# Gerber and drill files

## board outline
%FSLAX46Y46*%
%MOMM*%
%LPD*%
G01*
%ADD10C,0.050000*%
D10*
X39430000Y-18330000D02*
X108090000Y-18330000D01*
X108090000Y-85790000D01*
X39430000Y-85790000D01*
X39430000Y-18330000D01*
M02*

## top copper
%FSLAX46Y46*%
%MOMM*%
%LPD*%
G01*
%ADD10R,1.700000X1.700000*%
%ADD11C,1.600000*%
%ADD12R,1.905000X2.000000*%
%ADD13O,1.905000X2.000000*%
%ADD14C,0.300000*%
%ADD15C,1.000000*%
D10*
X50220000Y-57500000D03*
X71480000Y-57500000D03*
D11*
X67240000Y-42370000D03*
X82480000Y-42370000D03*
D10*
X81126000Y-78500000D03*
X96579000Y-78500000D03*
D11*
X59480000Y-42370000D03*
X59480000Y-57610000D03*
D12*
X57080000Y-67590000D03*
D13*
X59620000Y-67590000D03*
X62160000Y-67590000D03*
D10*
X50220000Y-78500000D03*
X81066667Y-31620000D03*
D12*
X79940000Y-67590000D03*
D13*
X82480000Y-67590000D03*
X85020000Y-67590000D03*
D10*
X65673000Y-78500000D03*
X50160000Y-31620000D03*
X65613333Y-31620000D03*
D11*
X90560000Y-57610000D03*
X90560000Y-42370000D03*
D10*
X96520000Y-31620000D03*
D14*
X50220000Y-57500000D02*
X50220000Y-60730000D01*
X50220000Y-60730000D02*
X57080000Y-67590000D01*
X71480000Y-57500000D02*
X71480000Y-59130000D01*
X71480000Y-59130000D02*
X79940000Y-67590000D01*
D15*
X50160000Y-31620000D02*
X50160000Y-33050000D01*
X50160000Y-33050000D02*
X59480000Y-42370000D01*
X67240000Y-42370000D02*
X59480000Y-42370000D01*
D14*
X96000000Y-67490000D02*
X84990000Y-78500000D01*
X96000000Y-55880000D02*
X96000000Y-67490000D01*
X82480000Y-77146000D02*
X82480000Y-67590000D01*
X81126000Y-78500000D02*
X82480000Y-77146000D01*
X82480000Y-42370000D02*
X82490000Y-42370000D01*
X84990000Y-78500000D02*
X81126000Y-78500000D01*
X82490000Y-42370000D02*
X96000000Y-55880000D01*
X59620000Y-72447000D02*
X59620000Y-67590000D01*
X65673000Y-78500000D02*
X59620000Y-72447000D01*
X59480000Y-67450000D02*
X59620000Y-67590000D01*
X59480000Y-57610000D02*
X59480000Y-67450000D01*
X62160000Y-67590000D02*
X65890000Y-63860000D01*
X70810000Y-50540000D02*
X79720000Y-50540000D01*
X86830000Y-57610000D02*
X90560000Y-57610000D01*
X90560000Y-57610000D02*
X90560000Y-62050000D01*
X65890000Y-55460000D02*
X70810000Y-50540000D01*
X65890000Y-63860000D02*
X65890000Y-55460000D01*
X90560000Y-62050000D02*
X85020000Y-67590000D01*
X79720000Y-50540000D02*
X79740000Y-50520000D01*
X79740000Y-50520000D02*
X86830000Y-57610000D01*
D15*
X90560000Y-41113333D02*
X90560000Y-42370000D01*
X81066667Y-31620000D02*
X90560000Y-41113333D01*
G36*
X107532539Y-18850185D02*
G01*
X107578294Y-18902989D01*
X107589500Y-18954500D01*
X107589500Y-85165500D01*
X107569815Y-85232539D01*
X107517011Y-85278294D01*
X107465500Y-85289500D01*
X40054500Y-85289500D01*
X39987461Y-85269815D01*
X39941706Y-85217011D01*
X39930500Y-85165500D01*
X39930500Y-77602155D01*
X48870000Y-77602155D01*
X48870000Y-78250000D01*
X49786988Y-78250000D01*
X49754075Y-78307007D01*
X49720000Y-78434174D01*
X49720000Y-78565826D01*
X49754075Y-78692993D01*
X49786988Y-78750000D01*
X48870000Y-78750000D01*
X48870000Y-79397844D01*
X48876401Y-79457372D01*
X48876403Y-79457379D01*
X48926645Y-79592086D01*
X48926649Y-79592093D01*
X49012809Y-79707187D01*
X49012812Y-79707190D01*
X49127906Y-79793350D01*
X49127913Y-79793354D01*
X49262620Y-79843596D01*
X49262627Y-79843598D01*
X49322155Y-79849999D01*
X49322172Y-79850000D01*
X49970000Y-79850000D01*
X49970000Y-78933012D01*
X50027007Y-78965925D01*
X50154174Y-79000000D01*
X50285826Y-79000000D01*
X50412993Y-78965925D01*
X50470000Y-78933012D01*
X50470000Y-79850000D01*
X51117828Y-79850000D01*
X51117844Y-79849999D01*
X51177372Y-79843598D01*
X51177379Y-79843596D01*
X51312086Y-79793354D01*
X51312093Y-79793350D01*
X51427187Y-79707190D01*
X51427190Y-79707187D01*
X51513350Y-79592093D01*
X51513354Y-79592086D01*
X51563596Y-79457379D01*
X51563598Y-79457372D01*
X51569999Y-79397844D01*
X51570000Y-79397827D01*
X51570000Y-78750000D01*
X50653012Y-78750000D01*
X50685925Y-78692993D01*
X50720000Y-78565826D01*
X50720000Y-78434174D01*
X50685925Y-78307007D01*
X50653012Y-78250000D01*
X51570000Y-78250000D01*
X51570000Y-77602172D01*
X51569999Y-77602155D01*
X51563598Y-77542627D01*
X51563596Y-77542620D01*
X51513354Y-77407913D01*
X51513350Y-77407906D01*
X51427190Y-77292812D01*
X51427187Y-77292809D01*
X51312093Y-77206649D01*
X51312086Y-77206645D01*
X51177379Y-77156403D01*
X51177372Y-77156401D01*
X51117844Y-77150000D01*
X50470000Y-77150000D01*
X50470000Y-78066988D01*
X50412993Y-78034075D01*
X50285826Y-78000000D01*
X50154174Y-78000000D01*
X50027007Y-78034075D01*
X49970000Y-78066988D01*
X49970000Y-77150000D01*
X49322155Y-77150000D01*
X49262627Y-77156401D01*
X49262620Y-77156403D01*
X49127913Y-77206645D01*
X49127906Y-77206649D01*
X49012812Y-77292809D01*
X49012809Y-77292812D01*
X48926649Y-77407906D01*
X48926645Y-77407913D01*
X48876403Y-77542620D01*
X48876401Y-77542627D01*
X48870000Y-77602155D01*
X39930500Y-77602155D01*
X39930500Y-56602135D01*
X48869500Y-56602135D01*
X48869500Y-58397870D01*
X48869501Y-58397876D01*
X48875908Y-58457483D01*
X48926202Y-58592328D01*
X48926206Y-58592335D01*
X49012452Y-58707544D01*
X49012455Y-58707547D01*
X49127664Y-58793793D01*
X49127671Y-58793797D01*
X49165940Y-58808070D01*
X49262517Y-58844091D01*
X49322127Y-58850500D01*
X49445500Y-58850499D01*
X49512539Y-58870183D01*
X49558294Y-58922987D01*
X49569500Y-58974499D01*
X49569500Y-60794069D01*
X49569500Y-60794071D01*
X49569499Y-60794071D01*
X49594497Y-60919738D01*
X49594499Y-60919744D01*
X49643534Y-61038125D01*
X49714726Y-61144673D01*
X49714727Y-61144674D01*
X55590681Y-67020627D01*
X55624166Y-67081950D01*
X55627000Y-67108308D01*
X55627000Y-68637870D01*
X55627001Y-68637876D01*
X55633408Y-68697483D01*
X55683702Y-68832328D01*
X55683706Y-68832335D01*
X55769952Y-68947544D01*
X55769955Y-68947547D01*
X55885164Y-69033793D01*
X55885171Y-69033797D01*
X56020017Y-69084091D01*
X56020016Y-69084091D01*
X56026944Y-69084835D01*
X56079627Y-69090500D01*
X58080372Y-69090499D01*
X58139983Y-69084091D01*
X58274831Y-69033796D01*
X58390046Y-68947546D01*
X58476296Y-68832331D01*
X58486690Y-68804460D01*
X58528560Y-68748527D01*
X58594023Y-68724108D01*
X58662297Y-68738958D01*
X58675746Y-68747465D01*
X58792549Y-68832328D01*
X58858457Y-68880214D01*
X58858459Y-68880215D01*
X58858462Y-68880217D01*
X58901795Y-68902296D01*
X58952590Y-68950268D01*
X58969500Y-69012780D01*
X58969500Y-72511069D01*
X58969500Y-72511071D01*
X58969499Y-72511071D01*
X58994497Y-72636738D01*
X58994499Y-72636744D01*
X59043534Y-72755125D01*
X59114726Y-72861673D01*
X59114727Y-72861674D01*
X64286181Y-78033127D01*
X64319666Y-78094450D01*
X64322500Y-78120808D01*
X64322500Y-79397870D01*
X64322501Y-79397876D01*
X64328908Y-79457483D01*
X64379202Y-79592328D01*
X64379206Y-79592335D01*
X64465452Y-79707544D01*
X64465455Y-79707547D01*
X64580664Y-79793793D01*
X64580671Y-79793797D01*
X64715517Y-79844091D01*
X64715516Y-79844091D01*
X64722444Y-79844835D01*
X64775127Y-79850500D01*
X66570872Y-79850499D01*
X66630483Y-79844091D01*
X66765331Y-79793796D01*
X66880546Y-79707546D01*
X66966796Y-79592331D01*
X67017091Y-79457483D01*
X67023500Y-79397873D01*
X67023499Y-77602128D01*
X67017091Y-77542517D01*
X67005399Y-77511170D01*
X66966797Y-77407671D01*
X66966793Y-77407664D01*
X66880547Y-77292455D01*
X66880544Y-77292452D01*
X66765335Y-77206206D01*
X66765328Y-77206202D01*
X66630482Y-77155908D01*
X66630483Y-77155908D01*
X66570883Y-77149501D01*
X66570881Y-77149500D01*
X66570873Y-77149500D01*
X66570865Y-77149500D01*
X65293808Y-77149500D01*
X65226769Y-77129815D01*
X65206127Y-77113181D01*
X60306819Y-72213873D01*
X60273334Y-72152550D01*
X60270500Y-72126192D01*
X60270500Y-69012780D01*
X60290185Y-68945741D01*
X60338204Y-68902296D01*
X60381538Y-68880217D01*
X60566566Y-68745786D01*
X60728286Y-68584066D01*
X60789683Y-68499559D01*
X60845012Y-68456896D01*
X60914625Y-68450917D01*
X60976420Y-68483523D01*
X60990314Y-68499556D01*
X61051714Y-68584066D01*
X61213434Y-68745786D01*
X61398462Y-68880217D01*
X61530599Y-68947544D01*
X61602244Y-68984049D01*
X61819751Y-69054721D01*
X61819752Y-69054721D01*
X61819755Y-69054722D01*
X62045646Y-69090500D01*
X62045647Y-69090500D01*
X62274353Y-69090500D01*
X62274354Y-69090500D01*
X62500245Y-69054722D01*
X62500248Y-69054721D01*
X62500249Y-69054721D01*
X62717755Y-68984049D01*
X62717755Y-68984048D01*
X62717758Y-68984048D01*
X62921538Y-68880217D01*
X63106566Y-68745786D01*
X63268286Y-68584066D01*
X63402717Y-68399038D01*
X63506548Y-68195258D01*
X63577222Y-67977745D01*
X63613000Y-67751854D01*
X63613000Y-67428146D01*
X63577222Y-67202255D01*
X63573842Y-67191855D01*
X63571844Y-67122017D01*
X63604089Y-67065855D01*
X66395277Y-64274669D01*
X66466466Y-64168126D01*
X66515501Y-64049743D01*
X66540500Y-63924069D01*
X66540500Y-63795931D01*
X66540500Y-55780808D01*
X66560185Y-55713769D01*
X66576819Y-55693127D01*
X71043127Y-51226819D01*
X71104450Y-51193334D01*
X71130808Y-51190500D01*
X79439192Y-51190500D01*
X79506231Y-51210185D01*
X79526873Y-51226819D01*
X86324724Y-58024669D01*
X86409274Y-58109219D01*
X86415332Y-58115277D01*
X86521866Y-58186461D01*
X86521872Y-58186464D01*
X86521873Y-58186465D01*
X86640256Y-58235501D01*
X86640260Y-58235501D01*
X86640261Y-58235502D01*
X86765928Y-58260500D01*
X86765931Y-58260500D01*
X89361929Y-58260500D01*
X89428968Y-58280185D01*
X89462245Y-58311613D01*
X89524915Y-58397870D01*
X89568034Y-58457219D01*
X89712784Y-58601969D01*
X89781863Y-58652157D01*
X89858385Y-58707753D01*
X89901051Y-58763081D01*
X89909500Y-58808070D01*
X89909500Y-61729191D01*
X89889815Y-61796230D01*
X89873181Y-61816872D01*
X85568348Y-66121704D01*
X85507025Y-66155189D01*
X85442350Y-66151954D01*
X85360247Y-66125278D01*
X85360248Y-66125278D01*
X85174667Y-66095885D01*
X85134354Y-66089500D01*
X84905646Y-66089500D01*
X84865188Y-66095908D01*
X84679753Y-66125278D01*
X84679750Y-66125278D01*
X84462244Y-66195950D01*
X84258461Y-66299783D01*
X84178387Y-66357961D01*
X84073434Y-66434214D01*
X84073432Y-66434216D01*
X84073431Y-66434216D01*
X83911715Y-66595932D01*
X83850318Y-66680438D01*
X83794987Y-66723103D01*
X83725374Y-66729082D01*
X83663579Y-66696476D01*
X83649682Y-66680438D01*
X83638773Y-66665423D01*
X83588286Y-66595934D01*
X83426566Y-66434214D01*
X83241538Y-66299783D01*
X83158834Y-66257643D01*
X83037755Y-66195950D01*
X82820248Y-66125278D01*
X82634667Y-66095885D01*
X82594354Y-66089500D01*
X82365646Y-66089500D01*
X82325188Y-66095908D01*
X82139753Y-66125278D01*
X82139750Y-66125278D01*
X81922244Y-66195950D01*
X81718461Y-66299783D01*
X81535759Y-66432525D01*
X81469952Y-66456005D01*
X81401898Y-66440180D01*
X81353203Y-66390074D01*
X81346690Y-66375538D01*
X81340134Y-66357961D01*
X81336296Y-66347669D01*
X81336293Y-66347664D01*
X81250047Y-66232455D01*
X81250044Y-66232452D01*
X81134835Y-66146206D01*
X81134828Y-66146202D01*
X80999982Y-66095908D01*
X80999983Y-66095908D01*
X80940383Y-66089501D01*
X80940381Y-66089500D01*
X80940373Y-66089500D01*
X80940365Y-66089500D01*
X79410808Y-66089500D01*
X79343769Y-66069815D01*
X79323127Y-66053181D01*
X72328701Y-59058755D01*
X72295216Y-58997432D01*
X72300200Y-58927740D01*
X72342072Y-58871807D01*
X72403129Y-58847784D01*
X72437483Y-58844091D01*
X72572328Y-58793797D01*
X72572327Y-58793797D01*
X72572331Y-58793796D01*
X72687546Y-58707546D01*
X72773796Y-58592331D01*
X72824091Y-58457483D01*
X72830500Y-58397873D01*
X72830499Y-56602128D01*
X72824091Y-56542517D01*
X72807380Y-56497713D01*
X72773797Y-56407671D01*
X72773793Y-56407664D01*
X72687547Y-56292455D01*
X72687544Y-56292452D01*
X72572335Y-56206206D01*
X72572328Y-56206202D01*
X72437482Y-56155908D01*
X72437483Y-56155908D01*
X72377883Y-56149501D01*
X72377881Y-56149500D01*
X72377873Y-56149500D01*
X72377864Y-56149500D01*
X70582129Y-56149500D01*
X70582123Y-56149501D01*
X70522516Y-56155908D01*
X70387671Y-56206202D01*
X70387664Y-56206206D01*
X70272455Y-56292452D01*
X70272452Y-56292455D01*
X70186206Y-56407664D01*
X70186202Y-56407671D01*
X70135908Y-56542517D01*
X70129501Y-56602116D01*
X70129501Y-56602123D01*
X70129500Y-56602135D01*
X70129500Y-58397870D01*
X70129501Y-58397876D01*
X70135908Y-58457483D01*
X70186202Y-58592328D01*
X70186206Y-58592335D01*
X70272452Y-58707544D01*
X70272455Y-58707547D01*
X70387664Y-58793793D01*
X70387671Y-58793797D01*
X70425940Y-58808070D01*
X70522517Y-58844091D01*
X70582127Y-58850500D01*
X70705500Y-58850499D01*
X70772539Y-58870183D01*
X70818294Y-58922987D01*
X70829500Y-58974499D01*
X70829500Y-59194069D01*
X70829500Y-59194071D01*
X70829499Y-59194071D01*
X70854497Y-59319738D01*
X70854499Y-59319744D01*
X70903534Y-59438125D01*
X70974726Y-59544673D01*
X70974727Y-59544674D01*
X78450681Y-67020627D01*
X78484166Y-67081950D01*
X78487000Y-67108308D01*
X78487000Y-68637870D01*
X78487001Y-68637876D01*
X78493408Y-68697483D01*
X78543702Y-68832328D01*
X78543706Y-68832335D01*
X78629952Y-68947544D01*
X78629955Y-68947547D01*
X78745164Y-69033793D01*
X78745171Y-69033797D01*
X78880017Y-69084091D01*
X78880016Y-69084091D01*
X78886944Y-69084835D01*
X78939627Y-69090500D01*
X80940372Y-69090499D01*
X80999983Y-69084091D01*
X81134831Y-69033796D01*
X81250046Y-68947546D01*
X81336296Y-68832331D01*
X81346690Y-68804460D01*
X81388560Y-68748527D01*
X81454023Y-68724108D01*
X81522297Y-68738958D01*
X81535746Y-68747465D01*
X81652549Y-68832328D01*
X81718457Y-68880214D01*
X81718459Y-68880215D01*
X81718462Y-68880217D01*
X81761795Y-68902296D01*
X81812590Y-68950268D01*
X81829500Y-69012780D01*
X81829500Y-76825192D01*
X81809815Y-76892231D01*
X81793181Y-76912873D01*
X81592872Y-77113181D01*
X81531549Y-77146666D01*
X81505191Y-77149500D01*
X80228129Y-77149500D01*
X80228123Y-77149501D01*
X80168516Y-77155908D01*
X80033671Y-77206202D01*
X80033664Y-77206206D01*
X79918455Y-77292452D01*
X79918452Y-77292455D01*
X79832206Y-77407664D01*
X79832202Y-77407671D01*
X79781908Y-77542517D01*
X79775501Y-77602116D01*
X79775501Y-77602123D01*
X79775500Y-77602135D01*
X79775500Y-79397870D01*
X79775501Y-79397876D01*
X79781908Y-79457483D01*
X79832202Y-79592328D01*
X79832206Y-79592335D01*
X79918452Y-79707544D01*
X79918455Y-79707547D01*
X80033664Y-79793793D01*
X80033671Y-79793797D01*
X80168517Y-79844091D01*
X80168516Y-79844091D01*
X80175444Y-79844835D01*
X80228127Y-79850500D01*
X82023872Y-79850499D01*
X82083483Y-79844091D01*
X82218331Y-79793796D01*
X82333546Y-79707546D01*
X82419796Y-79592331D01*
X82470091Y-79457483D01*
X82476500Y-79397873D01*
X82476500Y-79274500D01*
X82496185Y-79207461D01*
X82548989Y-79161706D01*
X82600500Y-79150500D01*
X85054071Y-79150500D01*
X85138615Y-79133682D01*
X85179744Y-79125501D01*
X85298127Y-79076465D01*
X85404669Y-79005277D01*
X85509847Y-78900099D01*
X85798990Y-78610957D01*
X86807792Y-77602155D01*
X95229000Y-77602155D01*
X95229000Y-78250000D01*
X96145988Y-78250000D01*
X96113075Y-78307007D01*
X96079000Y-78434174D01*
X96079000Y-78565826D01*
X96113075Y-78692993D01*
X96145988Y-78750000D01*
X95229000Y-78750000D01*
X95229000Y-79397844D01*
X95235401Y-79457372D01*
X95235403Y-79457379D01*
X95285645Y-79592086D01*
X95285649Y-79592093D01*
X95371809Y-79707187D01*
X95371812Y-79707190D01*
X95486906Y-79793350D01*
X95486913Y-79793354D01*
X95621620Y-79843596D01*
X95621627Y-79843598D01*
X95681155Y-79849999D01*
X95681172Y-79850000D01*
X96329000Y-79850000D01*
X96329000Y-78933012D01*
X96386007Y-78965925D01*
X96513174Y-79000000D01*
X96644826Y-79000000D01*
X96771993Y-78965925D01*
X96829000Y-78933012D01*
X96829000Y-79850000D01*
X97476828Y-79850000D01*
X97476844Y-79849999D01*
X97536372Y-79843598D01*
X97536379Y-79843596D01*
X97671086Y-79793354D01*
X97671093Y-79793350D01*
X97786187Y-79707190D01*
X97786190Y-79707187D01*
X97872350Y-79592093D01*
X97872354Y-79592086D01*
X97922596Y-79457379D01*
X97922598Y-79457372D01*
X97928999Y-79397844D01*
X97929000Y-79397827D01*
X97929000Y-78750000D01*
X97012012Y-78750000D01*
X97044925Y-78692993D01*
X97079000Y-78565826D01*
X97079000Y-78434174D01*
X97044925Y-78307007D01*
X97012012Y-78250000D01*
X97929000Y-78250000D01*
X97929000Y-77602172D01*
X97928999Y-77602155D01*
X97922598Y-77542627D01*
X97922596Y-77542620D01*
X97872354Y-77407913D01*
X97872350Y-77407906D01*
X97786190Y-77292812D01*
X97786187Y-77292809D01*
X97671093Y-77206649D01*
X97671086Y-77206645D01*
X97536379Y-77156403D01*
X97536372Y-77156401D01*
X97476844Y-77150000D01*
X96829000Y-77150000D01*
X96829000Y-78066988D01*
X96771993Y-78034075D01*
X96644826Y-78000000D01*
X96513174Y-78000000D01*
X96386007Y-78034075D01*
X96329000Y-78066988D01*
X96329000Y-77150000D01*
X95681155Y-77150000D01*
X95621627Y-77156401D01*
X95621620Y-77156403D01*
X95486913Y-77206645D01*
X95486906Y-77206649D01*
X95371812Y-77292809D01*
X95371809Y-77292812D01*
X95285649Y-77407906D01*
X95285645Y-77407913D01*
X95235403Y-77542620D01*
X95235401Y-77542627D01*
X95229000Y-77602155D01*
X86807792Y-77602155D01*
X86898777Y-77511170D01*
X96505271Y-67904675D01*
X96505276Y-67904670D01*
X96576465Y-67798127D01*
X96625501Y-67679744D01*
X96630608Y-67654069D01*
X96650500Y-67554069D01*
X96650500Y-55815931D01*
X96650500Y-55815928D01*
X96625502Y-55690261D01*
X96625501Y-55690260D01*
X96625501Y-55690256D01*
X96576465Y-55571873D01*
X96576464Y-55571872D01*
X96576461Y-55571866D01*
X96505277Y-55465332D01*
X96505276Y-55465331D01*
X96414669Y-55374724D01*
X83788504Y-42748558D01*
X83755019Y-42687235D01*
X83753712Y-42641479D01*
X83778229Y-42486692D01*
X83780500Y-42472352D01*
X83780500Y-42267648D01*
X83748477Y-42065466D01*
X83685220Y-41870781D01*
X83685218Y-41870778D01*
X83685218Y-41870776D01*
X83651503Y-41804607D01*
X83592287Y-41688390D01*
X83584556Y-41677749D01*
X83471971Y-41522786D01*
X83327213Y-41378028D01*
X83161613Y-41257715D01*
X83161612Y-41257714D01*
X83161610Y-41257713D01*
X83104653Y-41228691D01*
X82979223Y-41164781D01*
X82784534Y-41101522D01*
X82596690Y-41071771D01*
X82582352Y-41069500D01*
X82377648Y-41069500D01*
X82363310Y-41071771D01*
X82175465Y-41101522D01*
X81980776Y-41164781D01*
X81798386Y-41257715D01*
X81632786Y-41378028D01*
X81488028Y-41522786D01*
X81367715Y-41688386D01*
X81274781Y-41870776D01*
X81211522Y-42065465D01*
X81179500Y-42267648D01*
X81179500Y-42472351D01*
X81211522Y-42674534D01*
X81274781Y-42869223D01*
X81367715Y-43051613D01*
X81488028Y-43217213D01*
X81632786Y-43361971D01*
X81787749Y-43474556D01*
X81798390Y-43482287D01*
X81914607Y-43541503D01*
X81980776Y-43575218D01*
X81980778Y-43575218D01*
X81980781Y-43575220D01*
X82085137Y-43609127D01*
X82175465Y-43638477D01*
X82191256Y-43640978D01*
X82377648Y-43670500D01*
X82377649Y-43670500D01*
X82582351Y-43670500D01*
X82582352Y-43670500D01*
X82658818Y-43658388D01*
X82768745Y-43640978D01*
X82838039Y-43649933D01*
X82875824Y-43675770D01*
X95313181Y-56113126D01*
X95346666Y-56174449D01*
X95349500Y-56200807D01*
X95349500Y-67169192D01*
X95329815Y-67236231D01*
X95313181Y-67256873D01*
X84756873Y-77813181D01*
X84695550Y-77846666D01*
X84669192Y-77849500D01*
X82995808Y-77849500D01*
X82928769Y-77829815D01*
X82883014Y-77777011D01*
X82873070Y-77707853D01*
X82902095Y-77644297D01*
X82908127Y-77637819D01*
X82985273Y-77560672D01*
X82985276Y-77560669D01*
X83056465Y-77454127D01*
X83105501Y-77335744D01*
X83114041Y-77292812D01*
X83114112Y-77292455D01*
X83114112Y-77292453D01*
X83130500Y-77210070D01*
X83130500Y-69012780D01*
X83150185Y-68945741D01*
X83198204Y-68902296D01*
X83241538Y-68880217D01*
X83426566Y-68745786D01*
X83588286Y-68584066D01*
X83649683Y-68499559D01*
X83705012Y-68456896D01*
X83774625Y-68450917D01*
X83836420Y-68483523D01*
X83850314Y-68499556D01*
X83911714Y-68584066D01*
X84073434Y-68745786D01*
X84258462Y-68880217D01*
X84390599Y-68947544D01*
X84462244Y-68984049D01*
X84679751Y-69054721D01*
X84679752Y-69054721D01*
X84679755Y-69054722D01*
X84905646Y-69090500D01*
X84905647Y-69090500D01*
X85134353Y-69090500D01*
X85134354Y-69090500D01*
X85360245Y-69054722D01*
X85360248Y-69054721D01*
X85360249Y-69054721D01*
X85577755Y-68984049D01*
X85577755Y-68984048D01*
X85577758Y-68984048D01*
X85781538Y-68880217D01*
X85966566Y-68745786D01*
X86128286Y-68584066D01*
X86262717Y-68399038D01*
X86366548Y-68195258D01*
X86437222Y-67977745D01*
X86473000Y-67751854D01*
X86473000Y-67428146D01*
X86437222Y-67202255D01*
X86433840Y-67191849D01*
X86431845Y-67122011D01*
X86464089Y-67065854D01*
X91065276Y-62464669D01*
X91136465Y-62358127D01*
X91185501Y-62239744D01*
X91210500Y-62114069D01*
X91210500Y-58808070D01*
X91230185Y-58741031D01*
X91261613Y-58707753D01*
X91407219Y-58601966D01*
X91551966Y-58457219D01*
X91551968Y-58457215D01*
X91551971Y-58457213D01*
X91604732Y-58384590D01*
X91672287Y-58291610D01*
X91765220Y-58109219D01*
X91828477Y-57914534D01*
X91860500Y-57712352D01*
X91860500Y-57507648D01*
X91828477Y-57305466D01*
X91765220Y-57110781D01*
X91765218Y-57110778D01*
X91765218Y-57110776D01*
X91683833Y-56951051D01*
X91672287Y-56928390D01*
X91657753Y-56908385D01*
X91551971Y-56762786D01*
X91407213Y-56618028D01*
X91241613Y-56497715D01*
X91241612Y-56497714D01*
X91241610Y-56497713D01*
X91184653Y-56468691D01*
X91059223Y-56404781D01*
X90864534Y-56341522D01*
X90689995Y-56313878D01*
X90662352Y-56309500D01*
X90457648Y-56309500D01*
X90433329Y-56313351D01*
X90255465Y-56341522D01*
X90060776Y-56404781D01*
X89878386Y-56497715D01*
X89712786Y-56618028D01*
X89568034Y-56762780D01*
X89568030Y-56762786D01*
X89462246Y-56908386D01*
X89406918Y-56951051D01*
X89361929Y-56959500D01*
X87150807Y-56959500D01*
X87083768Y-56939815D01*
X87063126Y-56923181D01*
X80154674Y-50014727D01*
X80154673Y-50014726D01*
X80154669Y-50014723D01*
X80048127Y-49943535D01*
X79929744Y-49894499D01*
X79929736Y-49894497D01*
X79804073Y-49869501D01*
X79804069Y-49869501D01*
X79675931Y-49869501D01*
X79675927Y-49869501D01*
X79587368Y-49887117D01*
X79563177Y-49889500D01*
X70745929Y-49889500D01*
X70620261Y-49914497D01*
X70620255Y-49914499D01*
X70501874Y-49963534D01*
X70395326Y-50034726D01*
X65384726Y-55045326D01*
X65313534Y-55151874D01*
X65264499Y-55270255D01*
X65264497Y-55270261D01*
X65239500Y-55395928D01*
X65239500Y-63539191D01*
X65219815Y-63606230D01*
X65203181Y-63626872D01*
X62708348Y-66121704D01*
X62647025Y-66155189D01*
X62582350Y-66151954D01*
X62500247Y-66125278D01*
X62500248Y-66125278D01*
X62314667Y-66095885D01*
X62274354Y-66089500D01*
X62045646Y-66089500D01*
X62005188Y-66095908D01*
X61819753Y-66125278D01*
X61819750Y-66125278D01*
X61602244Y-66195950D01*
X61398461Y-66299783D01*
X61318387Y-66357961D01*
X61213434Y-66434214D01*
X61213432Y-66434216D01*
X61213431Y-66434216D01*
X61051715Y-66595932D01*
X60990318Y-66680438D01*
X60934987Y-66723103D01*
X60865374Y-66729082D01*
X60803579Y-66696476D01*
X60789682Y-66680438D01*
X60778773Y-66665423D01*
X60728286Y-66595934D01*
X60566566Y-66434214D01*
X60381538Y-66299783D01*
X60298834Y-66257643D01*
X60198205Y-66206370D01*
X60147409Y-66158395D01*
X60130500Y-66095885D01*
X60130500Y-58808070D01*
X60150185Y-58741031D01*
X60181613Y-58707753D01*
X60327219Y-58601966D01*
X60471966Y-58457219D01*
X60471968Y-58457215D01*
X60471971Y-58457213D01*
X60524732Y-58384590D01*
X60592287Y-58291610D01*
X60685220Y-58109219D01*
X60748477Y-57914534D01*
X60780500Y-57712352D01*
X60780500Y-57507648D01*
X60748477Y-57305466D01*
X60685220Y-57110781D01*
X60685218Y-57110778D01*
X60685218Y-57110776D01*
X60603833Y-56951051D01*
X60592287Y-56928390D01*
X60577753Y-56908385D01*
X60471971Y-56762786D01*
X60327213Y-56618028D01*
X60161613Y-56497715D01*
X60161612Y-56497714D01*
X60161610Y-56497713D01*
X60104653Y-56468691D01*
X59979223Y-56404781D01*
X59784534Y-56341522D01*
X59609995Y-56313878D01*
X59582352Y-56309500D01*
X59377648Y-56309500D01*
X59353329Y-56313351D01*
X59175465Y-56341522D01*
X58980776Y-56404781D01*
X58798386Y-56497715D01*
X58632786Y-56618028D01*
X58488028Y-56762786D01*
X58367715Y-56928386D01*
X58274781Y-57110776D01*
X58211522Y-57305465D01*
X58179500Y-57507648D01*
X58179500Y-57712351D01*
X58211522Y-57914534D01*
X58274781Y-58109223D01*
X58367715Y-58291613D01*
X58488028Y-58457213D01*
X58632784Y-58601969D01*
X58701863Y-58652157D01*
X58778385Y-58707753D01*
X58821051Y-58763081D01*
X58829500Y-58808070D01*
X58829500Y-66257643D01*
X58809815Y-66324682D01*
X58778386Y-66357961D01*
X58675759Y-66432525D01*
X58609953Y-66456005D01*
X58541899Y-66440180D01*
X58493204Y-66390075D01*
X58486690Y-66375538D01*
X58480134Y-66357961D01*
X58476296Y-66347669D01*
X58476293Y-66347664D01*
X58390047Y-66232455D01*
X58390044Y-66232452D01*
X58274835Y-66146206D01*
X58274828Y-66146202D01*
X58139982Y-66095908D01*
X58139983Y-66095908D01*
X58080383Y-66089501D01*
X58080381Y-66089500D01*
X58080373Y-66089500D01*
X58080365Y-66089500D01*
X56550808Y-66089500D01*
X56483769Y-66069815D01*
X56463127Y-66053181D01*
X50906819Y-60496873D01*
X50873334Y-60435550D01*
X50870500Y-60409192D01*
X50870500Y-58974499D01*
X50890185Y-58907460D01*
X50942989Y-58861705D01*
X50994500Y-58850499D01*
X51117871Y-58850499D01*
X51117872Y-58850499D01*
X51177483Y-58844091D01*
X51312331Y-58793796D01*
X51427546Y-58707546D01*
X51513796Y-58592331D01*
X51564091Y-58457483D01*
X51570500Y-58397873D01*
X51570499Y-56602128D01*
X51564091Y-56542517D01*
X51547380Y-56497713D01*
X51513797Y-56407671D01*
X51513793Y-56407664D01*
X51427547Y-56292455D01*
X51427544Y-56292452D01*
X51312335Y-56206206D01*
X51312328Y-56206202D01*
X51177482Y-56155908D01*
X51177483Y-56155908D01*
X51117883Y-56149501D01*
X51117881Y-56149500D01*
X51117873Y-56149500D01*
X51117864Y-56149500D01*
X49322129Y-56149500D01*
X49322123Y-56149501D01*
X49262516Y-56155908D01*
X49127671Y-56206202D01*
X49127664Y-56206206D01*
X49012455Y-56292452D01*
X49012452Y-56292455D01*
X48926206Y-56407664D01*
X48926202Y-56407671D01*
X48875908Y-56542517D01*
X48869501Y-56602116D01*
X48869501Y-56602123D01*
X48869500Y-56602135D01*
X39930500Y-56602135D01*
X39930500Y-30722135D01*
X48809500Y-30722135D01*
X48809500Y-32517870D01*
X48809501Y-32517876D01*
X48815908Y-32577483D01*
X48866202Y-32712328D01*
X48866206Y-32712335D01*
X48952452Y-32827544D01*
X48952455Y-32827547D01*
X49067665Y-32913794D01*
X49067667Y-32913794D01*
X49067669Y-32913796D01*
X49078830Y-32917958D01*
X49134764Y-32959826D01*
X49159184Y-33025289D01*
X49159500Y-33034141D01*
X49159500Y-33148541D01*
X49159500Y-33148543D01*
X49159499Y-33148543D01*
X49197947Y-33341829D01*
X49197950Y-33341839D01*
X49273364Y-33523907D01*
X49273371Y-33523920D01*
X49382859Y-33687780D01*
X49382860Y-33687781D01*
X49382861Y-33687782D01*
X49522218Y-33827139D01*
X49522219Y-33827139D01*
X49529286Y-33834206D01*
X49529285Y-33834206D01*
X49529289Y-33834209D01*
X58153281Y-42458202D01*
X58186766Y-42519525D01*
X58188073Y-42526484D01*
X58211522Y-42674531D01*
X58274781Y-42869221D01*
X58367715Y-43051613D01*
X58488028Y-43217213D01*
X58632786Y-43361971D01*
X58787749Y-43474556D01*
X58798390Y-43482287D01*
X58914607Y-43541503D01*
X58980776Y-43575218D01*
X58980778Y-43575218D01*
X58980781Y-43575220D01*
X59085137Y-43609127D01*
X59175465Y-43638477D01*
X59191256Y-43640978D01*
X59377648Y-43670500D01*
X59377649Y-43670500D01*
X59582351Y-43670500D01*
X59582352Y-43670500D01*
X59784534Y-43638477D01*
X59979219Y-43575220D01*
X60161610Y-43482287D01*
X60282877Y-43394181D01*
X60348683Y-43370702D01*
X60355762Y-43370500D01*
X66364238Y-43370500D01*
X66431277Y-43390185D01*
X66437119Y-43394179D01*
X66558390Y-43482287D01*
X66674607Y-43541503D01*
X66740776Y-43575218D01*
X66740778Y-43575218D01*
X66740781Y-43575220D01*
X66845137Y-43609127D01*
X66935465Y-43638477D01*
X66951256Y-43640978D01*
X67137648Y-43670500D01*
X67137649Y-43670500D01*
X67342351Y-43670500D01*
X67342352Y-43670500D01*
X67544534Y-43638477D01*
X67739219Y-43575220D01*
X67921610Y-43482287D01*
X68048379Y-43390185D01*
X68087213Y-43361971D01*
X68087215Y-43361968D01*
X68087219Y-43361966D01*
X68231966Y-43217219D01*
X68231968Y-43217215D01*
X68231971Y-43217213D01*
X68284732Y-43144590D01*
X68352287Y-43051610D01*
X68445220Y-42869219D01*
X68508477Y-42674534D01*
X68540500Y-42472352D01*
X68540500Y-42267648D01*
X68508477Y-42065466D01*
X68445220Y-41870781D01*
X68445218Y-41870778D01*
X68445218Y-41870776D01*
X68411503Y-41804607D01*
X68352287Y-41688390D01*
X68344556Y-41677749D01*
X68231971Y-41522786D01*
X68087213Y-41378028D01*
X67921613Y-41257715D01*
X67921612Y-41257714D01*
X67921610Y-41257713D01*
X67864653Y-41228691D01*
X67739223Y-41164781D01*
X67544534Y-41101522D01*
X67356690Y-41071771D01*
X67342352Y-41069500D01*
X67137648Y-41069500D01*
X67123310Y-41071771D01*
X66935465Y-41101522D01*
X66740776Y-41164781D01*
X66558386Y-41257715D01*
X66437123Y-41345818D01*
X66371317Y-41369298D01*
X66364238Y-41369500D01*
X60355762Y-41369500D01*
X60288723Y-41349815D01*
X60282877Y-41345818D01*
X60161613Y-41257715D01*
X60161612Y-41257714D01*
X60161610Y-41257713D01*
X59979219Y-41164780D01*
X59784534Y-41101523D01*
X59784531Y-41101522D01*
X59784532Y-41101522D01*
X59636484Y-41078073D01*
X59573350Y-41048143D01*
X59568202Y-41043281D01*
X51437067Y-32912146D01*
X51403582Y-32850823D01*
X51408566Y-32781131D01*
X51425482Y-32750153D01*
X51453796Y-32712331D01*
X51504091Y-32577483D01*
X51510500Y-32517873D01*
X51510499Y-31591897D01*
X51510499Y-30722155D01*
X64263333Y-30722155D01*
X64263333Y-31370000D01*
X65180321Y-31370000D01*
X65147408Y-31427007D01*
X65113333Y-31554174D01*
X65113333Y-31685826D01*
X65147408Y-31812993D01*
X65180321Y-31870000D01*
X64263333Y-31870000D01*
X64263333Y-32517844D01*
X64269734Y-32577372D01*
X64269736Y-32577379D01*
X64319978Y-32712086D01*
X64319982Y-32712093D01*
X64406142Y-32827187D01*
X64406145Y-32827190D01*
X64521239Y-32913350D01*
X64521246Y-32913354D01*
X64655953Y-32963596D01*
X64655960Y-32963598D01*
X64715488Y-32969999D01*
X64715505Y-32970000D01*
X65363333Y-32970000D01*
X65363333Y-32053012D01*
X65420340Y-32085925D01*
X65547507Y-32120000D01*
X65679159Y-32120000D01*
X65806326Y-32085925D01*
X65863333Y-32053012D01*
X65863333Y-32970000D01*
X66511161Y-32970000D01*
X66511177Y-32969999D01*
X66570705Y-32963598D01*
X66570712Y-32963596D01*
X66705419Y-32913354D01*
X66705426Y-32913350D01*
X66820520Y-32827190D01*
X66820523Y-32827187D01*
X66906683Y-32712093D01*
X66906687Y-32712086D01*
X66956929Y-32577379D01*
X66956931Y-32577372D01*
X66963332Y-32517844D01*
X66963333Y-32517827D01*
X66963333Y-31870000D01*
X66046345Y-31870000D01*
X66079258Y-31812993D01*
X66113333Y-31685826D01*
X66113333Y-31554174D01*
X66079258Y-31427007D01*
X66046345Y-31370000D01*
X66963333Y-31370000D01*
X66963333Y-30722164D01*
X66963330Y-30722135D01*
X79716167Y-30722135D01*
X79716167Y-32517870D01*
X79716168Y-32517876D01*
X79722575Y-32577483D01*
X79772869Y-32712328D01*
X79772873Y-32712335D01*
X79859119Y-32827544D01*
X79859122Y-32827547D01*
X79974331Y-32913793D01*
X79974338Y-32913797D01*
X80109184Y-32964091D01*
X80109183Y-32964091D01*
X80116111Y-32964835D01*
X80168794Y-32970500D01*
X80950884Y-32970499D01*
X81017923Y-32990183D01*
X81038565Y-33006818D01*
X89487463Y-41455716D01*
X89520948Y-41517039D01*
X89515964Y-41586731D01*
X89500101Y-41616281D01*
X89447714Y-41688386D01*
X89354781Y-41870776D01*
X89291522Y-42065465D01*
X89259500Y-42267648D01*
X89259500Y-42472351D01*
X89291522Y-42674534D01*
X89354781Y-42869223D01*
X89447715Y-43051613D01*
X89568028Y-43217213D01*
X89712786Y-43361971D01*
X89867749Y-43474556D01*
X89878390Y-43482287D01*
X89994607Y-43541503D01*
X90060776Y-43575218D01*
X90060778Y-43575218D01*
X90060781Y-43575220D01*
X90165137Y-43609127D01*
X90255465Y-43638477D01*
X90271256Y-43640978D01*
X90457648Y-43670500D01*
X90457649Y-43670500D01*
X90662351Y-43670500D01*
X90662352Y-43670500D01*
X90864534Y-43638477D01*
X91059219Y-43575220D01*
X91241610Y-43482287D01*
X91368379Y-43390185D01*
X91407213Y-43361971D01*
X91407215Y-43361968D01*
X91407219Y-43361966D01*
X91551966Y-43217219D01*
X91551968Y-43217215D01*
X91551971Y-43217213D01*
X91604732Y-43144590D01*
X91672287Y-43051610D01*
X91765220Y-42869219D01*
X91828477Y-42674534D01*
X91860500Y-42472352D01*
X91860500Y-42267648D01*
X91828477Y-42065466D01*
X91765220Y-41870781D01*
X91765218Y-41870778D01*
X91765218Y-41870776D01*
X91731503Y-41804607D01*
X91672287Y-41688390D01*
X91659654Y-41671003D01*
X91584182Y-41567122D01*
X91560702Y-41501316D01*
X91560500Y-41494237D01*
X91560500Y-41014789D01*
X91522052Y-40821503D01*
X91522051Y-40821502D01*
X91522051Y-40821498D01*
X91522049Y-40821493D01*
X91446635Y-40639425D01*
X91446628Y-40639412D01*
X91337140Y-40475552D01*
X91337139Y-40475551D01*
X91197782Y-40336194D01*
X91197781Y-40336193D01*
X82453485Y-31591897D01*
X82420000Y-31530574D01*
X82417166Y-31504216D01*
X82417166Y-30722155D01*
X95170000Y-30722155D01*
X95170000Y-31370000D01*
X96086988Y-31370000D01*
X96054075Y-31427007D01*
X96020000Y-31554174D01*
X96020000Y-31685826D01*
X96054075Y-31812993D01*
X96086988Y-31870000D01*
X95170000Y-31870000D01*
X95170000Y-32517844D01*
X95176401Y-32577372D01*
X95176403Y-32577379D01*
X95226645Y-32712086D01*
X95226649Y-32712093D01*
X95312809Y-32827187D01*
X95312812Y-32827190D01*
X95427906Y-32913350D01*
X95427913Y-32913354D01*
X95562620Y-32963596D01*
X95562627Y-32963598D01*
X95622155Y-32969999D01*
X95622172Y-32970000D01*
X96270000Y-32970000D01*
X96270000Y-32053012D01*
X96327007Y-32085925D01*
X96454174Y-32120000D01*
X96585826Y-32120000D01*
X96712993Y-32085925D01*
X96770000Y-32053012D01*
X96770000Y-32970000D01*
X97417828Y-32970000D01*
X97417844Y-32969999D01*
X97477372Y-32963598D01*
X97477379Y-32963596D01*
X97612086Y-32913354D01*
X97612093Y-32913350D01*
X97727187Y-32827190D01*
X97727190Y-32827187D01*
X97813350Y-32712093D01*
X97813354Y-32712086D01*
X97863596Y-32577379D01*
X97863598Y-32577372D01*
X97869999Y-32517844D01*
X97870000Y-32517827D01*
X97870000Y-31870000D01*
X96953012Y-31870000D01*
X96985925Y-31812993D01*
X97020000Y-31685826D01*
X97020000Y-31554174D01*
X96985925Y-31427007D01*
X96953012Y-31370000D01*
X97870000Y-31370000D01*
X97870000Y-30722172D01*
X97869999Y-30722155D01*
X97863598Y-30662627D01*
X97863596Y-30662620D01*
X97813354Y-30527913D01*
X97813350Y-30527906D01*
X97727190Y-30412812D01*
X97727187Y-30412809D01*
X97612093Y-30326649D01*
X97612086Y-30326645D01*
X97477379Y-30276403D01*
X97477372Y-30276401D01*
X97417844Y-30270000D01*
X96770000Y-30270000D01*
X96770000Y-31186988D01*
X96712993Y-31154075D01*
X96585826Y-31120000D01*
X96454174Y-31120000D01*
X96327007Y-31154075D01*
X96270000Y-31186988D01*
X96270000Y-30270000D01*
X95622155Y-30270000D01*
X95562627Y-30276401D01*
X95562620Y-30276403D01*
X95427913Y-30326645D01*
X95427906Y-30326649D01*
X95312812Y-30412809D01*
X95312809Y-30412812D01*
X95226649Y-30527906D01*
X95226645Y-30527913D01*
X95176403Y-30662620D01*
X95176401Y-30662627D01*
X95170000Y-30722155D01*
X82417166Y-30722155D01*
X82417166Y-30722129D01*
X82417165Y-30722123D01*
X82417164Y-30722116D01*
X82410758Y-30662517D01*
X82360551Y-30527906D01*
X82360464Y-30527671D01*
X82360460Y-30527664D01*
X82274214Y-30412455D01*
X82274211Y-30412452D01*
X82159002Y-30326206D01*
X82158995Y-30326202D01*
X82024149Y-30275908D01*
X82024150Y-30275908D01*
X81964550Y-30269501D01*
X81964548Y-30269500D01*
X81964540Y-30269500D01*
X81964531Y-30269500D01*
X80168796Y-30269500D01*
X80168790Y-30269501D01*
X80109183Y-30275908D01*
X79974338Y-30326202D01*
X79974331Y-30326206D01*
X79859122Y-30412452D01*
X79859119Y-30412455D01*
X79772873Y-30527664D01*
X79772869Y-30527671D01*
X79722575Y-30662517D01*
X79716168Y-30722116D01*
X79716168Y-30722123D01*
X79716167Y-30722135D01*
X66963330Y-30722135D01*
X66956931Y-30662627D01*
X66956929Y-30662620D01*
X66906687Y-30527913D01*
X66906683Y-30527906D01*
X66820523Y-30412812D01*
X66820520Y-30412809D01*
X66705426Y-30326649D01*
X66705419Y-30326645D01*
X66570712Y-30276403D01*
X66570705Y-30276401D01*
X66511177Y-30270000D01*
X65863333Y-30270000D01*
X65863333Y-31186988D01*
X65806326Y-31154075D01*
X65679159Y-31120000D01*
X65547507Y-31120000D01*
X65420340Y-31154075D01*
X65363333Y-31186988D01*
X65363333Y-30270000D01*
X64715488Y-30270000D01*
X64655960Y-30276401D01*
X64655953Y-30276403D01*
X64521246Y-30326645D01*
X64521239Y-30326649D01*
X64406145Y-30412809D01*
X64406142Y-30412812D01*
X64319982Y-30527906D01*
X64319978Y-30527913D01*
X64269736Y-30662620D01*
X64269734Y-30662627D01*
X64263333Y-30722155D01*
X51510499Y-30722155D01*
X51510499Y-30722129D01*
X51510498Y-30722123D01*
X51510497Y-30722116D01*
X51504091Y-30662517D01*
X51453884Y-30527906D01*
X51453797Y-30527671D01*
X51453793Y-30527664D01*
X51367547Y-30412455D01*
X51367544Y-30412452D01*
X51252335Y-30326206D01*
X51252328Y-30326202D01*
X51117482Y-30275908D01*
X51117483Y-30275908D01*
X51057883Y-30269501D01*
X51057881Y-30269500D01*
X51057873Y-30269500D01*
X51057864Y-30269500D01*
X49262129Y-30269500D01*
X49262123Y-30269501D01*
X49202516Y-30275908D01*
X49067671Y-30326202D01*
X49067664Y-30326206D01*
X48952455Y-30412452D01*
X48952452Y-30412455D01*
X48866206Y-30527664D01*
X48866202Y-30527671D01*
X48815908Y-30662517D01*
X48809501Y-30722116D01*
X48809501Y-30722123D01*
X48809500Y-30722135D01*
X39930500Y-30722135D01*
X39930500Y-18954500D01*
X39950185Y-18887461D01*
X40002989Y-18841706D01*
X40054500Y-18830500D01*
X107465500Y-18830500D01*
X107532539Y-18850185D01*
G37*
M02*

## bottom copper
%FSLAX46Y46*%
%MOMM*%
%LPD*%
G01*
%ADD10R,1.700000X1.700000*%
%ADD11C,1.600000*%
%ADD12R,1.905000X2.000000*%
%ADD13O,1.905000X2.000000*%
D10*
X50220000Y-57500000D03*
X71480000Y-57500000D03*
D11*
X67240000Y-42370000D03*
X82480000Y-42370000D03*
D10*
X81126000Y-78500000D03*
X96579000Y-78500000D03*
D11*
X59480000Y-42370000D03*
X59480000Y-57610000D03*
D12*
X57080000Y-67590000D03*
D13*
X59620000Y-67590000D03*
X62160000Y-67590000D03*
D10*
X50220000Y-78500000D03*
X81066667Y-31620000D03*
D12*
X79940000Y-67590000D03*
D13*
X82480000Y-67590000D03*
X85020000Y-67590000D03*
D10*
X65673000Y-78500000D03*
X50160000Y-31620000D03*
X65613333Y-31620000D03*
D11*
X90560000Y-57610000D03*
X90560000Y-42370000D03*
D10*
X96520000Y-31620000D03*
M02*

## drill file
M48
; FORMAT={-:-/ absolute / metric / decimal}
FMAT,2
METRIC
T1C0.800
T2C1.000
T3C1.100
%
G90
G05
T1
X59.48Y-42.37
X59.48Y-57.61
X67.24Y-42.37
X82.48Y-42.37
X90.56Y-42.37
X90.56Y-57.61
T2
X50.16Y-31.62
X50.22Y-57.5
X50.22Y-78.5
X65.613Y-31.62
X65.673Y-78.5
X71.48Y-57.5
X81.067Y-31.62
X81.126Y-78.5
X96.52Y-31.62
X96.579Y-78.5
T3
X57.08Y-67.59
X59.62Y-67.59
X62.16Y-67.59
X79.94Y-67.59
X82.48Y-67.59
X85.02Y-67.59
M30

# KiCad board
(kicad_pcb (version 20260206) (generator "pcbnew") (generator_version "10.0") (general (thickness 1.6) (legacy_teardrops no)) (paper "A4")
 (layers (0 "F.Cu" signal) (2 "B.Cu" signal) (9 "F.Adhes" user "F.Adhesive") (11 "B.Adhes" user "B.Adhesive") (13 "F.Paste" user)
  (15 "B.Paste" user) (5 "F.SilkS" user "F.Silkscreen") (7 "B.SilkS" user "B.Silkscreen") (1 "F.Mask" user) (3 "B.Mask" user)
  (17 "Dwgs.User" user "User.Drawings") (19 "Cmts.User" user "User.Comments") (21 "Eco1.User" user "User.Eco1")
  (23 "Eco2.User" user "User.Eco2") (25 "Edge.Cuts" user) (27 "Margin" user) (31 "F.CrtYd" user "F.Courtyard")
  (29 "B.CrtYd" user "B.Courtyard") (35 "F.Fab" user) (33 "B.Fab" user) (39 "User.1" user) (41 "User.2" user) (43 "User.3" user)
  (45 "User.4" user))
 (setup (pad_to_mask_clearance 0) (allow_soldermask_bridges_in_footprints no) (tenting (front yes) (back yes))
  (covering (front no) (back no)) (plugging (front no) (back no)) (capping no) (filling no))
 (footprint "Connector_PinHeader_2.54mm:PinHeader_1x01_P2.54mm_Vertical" (layer "F.Cu") (at 50.22 57.5 90)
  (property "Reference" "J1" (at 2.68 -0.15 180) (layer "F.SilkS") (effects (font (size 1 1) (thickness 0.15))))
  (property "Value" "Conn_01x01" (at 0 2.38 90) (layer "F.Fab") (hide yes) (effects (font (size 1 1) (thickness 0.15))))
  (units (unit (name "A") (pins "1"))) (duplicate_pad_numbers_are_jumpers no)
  (pad "1" thru_hole rect (at 0 0 90) (size 1.7 1.7) (drill 1) (layers "*.Cu" "*.Mask") (remove_unused_layers no) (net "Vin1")))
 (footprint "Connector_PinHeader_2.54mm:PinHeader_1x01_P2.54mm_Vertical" (layer "F.Cu") (at 71.48 57.5 -90)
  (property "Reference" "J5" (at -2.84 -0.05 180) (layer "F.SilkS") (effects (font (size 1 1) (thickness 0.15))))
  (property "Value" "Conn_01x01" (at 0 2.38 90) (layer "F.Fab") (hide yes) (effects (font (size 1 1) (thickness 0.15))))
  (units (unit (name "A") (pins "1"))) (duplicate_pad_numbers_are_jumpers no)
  (pad "1" thru_hole rect (at 0 0 270) (size 1.7 1.7) (drill 1) (layers "*.Cu" "*.Mask") (remove_unused_layers no) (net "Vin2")))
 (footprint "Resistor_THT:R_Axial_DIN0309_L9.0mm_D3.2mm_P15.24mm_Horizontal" (layer "F.Cu") (at 67.24 42.37)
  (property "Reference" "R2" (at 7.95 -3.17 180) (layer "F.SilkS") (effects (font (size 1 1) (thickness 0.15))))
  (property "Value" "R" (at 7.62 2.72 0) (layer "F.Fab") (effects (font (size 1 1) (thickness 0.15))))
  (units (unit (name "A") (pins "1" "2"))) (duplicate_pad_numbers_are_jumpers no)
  (pad "1" thru_hole circle (at 0 0) (size 1.6 1.6) (drill 0.8) (layers "*.Cu" "*.Mask") (remove_unused_layers no) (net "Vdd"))
  (pad "2" thru_hole circle (at 15.24 0) (size 1.6 1.6) (drill 0.8) (layers "*.Cu" "*.Mask") (remove_unused_layers no) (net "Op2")))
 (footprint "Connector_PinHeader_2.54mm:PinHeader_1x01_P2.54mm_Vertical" (layer "F.Cu") (at 81.126 78.5)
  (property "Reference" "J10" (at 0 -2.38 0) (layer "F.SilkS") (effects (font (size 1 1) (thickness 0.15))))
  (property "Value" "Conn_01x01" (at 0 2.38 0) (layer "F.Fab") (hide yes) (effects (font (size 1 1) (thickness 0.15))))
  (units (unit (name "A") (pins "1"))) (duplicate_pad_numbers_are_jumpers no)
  (pad "1" thru_hole rect (at 0 0) (size 1.7 1.7) (drill 1) (layers "*.Cu" "*.Mask") (remove_unused_layers no) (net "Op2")))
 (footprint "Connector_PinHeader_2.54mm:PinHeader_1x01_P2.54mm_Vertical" (layer "F.Cu") (at 96.579 78.5 -90)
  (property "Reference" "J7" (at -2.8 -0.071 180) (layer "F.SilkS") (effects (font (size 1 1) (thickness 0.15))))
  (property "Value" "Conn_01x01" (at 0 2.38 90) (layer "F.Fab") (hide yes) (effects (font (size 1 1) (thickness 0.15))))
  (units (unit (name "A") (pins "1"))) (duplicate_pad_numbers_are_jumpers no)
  (pad "1" thru_hole rect (at 0 0 270) (size 1.7 1.7) (drill 1) (layers "*.Cu" "*.Mask") (remove_unused_layers no) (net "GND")))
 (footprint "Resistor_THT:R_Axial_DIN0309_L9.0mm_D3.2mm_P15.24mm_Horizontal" (layer "F.Cu") (at 59.48 42.37 -90)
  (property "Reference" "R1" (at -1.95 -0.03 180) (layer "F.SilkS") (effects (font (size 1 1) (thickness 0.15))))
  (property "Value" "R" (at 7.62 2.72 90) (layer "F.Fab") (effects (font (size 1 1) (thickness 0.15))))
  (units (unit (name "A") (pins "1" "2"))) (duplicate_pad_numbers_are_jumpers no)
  (pad "1" thru_hole circle (at 0 0 270) (size 1.6 1.6) (drill 0.8) (layers "*.Cu" "*.Mask") (remove_unused_layers no) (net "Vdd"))
  (pad "2" thru_hole circle (at 15.24 0 270) (size 1.6 1.6) (drill 0.8) (layers "*.Cu" "*.Mask") (remove_unused_layers no) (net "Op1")))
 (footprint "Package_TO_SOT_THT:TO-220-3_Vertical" (layer "F.Cu") (at 57.08 67.59)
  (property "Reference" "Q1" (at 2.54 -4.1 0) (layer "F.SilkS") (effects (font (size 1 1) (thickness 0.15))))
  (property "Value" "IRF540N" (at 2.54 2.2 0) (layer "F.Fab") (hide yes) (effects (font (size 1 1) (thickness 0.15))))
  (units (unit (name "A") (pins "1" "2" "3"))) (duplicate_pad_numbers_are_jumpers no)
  (pad "1" thru_hole rect (at 0 0) (size 1.905 2) (drill 1.1) (layers "*.Cu" "*.Mask") (remove_unused_layers no) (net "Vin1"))
  (pad "2" thru_hole oval (at 2.54 0) (size 1.905 2) (drill 1.1) (layers "*.Cu" "*.Mask") (remove_unused_layers no) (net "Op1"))
  (pad "3" thru_hole oval (at 5.08 0) (size 1.905 2) (drill 1.1) (layers "*.Cu" "*.Mask") (remove_unused_layers no) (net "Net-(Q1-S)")))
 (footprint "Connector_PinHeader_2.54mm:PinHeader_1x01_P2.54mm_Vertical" (layer "F.Cu") (at 50.22 78.5 90)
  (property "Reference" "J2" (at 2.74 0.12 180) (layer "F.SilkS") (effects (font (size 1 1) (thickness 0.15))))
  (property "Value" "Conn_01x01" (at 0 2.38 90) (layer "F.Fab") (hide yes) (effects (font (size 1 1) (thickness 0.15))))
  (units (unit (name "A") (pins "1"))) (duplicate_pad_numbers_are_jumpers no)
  (pad "1" thru_hole rect (at 0 0 90) (size 1.7 1.7) (drill 1) (layers "*.Cu" "*.Mask") (remove_unused_layers no) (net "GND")))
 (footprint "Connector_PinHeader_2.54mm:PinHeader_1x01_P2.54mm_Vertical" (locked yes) (layer "F.Cu") (at 81.066667 31.62)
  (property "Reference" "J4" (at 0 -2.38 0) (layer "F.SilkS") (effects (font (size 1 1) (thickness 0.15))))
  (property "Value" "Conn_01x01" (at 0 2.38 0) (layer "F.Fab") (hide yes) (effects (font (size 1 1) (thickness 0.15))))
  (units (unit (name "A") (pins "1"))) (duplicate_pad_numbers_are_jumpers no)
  (pad "1" thru_hole rect (at 0 0) (size 1.7 1.7) (drill 1) (layers "*.Cu" "*.Mask") (remove_unused_layers no) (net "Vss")))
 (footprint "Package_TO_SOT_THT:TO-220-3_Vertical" (layer "F.Cu") (at 79.94 67.59)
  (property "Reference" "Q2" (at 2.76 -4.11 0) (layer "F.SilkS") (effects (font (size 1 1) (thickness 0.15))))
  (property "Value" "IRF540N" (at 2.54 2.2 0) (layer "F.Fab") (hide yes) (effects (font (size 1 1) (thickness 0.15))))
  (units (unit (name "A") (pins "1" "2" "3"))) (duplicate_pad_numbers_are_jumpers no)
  (pad "1" thru_hole rect (at 0 0) (size 1.905 2) (drill 1.1) (layers "*.Cu" "*.Mask") (remove_unused_layers no) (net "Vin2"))
  (pad "2" thru_hole oval (at 2.54 0) (size 1.905 2) (drill 1.1) (layers "*.Cu" "*.Mask") (remove_unused_layers no) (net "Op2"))
  (pad "3" thru_hole oval (at 5.08 0) (size 1.905 2) (drill 1.1) (layers "*.Cu" "*.Mask") (remove_unused_layers no) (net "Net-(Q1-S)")))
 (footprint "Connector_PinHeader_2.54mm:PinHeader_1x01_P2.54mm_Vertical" (layer "F.Cu") (at 65.673 78.5)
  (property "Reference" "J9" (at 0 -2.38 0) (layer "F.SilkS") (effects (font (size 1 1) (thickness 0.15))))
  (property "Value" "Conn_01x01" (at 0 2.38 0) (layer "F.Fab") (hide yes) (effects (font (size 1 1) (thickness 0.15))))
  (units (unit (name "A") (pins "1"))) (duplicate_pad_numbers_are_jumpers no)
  (pad "1" thru_hole rect (at 0 0) (size 1.7 1.7) (drill 1) (layers "*.Cu" "*.Mask") (remove_unused_layers no) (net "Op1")))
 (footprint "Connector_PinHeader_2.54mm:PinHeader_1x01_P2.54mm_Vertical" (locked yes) (layer "F.Cu") (at 50.16 31.62)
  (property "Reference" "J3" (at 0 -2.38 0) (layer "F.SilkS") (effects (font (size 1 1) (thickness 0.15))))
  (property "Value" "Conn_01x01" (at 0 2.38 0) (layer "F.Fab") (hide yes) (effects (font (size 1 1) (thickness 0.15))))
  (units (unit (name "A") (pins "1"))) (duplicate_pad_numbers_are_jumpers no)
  (pad "1" thru_hole rect (at 0 0) (size 1.7 1.7) (drill 1) (layers "*.Cu" "*.Mask") (remove_unused_layers no) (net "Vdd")))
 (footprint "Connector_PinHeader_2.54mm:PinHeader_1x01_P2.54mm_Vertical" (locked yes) (layer "F.Cu") (at 65.613333 31.62)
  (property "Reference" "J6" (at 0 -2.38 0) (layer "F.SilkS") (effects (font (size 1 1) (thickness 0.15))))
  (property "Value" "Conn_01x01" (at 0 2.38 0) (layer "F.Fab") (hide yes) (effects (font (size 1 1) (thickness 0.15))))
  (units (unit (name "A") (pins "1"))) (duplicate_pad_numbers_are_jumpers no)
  (pad "1" thru_hole rect (at 0 0) (size 1.7 1.7) (drill 1) (layers "*.Cu" "*.Mask") (remove_unused_layers no) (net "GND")))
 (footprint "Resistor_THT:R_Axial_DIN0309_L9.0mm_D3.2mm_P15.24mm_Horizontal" (layer "F.Cu") (at 90.56 57.61 90)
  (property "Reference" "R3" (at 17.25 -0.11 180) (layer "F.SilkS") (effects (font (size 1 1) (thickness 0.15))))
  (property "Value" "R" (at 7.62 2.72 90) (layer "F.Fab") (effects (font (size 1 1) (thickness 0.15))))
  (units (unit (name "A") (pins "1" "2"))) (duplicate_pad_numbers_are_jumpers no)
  (pad "1" thru_hole circle (at 0 0 90) (size 1.6 1.6) (drill 0.8) (layers "*.Cu" "*.Mask") (remove_unused_layers no) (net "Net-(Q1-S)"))
  (pad "2" thru_hole circle (at 15.24 0 90) (size 1.6 1.6) (drill 0.8) (layers "*.Cu" "*.Mask") (remove_unused_layers no) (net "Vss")))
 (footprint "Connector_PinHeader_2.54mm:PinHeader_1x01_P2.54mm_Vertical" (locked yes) (layer "F.Cu") (at 96.52 31.62)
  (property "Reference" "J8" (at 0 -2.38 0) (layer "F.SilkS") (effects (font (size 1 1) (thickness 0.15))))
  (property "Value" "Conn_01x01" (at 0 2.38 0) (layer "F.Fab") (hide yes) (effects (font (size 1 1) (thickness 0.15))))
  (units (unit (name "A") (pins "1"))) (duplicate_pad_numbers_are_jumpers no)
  (pad "1" thru_hole rect (at 0 0) (size 1.7 1.7) (drill 1) (layers "*.Cu" "*.Mask") (remove_unused_layers no) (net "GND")))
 (gr_rect (start 39.43 18.33) (end 108.09 85.79) (stroke (width 0.05) (type default)) (fill no) (layer "Edge.Cuts"))
 (segment (start 50.22 57.5) (end 50.22 60.73) (width 0.3) (layer "F.Cu") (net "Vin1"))
 (segment (start 50.22 60.73) (end 57.08 67.59) (width 0.3) (layer "F.Cu") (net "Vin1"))
 (segment (start 71.48 57.5) (end 71.48 59.13) (width 0.3) (layer "F.Cu") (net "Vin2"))
 (segment (start 71.48 59.13) (end 79.94 67.59) (width 0.3) (layer "F.Cu") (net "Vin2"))
 (segment (start 50.16 31.62) (end 50.16 33.05) (width 1) (layer "F.Cu") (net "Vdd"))
 (segment (start 50.16 33.05) (end 59.48 42.37) (width 1) (layer "F.Cu") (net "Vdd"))
 (segment (start 67.24 42.37) (end 59.48 42.37) (width 1) (layer "F.Cu") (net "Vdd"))
 (segment (start 96 67.49) (end 84.99 78.5) (width 0.3) (layer "F.Cu") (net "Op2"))
 (segment (start 96 55.88) (end 96 67.49) (width 0.3) (layer "F.Cu") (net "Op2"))
 (segment (start 82.48 77.146) (end 82.48 67.59) (width 0.3) (layer "F.Cu") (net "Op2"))
 (segment (start 81.126 78.5) (end 82.48 77.146) (width 0.3) (layer "F.Cu") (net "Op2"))
 (segment (start 82.48 42.37) (end 82.49 42.37) (width 0.3) (layer "F.Cu") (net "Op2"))
 (segment (start 84.99 78.5) (end 81.126 78.5) (width 0.3) (layer "F.Cu") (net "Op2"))
 (segment (start 82.49 42.37) (end 96 55.88) (width 0.3) (layer "F.Cu") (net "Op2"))
 (segment (start 59.62 72.447) (end 59.62 67.59) (width 0.3) (layer "F.Cu") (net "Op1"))
 (segment (start 65.673 78.5) (end 59.62 72.447) (width 0.3) (layer "F.Cu") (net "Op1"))
 (segment (start 59.48 67.45) (end 59.62 67.59) (width 0.3) (layer "F.Cu") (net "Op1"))
 (segment (start 59.48 57.61) (end 59.48 67.45) (width 0.3) (layer "F.Cu") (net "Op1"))
 (segment (start 62.16 67.59) (end 65.89 63.86) (width 0.3) (layer "F.Cu") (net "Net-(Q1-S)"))
 (segment (start 70.81 50.54) (end 79.72 50.54) (width 0.3) (layer "F.Cu") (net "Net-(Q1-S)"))
 (segment (start 86.83 57.61) (end 90.56 57.61) (width 0.3) (layer "F.Cu") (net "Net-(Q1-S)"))
 (segment (start 90.56 57.61) (end 90.56 62.05) (width 0.3) (layer "F.Cu") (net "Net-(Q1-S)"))
 (segment (start 65.89 55.46) (end 70.81 50.54) (width 0.3) (layer "F.Cu") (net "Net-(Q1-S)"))
 (segment (start 65.89 63.86) (end 65.89 55.46) (width 0.3) (layer "F.Cu") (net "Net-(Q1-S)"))
 (segment (start 90.56 62.05) (end 85.02 67.59) (width 0.3) (layer "F.Cu") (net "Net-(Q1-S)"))
 (segment (start 79.72 50.54) (end 79.74 50.52) (width 0.3) (layer "F.Cu") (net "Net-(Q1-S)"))
 (segment (start 79.74 50.52) (end 86.83 57.61) (width 0.3) (layer "F.Cu") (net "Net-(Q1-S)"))
 (segment (start 90.56 41.113333) (end 90.56 42.37) (width 1) (layer "F.Cu") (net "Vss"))
 (segment (start 81.066667 31.62) (end 90.56 41.113333) (width 1) (layer "F.Cu") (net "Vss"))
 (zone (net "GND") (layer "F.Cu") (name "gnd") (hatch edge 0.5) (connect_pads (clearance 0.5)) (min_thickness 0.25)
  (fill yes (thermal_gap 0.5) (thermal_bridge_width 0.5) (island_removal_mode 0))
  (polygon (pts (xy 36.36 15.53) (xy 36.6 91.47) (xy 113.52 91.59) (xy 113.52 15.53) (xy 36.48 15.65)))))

